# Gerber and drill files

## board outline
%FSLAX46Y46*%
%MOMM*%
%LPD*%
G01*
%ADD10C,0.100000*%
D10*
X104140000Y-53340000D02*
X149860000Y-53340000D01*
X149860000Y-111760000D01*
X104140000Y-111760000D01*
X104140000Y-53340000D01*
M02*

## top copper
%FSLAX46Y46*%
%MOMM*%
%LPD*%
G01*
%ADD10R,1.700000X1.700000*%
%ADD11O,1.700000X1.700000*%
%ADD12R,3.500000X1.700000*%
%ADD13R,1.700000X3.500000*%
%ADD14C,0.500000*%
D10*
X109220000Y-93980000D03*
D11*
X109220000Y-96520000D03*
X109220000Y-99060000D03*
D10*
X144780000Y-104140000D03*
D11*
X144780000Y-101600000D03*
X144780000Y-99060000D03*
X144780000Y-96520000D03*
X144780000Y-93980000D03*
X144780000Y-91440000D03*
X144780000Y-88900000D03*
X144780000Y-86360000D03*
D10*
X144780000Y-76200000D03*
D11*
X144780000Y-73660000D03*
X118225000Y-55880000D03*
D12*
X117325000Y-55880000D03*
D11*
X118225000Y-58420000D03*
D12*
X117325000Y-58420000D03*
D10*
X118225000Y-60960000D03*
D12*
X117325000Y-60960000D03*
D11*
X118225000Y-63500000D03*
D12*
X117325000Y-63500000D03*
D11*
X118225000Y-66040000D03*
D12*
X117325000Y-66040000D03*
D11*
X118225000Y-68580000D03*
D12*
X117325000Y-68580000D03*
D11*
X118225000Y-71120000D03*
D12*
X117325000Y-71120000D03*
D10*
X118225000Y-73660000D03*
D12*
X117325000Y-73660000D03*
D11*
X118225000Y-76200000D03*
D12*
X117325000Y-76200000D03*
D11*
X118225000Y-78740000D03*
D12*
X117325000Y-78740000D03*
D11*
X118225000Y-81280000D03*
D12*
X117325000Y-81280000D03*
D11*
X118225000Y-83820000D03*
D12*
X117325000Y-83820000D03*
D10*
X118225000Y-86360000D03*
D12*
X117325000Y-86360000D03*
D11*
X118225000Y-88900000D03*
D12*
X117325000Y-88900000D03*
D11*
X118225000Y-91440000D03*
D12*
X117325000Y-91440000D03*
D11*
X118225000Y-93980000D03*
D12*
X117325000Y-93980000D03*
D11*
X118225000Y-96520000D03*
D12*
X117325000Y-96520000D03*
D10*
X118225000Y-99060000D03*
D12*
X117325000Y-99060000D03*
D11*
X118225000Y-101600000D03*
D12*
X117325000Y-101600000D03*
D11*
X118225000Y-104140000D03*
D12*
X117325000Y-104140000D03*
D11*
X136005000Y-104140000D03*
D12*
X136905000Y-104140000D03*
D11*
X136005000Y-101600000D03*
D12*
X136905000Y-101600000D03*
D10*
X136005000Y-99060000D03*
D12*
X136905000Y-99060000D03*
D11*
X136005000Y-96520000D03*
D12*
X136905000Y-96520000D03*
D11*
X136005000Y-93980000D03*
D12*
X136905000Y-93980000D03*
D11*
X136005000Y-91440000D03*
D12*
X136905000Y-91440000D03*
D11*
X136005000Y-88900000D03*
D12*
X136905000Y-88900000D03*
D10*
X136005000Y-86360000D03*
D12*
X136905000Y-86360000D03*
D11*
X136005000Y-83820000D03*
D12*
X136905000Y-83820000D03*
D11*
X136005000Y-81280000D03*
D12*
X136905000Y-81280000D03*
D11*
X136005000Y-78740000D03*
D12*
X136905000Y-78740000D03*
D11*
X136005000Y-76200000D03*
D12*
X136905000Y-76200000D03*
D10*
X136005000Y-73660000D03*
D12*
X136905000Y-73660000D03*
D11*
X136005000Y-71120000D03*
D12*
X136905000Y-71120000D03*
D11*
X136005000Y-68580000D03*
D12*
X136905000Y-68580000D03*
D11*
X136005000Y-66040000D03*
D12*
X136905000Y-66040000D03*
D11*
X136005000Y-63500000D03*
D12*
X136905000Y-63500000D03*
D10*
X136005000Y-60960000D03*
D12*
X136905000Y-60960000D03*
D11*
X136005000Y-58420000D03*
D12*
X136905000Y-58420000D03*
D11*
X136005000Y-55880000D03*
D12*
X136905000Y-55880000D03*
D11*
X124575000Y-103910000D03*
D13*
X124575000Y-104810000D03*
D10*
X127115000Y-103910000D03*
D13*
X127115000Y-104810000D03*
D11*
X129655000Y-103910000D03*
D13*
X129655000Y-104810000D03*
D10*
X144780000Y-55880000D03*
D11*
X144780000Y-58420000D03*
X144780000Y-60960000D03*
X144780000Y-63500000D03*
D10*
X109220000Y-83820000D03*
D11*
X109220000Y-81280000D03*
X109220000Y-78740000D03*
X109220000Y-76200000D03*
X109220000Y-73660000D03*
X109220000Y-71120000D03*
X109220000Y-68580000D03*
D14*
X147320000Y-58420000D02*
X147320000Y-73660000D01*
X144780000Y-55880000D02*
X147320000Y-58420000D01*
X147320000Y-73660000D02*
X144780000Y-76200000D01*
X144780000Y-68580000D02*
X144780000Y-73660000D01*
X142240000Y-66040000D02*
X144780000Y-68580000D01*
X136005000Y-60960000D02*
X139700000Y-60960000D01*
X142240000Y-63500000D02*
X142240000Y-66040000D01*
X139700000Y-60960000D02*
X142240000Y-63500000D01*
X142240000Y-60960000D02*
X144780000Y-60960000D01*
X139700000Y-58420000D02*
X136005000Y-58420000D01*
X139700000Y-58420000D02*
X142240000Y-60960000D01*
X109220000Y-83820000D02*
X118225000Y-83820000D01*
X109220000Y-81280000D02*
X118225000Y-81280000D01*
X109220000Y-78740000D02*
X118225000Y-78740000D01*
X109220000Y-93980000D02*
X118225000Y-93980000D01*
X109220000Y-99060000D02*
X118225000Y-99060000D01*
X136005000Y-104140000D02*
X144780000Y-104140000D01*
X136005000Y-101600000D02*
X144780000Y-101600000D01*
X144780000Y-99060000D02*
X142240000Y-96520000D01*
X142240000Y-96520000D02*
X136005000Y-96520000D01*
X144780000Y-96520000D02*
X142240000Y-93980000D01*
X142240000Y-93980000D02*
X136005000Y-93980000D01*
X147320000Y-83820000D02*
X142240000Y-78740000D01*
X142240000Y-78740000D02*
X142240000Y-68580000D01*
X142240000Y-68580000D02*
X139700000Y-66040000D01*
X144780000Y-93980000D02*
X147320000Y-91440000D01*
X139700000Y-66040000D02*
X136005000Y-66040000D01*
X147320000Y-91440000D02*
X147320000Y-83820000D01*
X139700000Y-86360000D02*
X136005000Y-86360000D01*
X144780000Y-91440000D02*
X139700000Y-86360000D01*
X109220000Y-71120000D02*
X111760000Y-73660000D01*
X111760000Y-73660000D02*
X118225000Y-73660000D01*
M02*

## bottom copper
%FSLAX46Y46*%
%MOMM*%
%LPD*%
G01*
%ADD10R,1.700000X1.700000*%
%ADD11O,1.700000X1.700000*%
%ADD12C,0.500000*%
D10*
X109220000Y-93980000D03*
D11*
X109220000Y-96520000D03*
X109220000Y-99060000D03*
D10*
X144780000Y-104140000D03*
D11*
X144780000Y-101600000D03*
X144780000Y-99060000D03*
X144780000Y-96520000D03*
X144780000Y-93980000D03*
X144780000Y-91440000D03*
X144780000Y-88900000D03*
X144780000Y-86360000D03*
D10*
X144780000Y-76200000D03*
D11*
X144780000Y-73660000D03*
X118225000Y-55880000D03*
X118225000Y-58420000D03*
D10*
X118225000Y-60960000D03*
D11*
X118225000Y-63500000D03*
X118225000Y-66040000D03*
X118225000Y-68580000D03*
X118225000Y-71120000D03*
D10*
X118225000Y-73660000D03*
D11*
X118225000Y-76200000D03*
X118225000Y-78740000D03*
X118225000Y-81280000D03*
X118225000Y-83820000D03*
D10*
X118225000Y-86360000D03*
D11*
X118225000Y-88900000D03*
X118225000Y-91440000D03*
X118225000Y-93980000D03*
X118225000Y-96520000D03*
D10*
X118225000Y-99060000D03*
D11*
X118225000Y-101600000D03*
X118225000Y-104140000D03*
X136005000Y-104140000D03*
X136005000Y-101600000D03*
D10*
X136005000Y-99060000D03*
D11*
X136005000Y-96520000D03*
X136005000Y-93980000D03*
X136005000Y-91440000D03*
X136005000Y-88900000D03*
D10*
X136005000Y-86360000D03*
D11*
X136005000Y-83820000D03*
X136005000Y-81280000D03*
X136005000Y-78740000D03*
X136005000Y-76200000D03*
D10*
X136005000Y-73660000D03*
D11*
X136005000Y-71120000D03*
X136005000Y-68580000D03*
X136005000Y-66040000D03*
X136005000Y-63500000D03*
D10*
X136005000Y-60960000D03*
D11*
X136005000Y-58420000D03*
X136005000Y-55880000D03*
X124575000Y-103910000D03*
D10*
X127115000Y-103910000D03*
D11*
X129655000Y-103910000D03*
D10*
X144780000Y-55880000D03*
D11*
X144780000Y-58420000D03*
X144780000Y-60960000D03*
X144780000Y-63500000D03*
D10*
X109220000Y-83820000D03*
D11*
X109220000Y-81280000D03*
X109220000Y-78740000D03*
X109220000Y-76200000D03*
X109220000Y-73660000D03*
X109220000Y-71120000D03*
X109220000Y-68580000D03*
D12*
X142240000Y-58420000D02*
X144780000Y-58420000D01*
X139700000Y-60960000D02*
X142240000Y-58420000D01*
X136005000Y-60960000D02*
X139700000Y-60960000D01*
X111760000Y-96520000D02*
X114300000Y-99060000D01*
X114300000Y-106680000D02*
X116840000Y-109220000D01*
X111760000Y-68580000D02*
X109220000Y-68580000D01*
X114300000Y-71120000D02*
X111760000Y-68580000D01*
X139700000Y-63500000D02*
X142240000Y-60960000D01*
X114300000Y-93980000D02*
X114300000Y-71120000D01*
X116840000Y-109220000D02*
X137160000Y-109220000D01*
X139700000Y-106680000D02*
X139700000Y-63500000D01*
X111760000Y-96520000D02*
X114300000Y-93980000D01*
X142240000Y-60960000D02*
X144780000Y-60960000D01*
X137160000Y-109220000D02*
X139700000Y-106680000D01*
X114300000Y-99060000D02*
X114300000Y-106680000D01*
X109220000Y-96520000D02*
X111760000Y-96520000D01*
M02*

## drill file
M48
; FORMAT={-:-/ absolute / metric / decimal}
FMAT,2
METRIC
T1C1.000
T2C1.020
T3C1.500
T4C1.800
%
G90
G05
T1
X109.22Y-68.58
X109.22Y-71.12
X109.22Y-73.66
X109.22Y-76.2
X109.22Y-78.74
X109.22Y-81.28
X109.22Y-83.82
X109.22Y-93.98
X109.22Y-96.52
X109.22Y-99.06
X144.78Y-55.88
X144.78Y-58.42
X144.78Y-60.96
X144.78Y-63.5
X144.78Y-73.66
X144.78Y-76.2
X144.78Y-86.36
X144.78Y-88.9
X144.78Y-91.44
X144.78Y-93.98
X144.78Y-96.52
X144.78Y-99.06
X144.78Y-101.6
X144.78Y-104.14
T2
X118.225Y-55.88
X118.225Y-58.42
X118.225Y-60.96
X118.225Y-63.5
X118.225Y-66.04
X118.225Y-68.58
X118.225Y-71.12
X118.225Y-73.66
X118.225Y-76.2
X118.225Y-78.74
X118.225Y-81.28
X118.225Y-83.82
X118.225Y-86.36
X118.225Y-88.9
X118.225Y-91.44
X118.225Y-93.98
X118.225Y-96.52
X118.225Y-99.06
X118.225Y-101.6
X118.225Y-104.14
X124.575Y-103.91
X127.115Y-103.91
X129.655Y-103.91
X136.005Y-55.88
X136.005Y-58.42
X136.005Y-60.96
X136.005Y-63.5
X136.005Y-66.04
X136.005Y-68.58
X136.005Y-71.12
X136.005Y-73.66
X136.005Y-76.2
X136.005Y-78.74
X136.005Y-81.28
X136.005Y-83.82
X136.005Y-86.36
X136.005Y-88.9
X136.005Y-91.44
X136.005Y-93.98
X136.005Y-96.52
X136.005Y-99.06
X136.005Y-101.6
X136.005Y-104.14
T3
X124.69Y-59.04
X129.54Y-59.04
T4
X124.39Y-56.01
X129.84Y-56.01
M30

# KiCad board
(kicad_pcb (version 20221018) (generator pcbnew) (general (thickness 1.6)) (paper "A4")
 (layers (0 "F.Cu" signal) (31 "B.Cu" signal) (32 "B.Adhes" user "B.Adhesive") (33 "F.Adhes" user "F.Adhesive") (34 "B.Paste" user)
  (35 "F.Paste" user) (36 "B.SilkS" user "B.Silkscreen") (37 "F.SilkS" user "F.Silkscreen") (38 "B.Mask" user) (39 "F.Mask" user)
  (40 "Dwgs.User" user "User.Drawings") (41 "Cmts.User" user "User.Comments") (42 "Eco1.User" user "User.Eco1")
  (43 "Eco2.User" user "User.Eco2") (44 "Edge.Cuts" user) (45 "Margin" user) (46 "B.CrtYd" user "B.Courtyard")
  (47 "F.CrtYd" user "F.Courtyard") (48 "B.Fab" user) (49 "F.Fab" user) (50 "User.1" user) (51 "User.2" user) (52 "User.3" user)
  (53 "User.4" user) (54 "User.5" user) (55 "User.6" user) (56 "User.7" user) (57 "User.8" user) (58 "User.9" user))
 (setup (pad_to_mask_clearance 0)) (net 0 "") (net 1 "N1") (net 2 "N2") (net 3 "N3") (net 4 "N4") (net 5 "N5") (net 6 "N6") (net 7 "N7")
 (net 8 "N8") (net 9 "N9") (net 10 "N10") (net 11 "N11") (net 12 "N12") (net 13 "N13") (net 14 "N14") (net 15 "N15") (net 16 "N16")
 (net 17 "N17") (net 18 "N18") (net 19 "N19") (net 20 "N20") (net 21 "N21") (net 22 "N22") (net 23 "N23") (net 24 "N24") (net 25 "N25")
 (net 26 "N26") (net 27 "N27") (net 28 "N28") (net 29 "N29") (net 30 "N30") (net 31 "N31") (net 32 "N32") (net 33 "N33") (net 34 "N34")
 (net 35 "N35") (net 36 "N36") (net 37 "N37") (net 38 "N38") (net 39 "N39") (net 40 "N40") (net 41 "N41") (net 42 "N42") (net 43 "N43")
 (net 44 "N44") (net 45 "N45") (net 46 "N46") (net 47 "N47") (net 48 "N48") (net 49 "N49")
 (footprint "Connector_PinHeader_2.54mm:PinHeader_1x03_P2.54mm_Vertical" (layer "F.Cu") (at 109.22 93.98)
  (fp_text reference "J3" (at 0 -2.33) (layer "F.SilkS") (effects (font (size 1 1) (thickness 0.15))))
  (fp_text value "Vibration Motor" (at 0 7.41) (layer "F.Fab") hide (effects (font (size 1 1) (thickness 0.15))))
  (pad "1" thru_hole rect (at 0 0) (size 1.7 1.7) (drill 1) (layers "*.Cu" "*.Mask") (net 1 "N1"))
  (pad "2" thru_hole oval (at 0 2.54) (size 1.7 1.7) (drill 1) (layers "*.Cu" "*.Mask") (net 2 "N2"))
  (pad "3" thru_hole oval (at 0 5.08) (size 1.7 1.7) (drill 1) (layers "*.Cu" "*.Mask") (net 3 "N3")))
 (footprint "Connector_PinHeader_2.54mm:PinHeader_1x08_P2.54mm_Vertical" (layer "F.Cu") (at 144.78 104.14 180)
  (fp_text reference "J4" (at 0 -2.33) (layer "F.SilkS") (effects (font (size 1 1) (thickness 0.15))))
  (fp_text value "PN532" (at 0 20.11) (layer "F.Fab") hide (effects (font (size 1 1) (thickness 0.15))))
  (pad "1" thru_hole rect (at 0 0 180) (size 1.7 1.7) (drill 1) (layers "*.Cu" "*.Mask") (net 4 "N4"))
  (pad "2" thru_hole oval (at 0 2.54 180) (size 1.7 1.7) (drill 1) (layers "*.Cu" "*.Mask") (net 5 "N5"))
  (pad "3" thru_hole oval (at 0 5.08 180) (size 1.7 1.7) (drill 1) (layers "*.Cu" "*.Mask") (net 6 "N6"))
  (pad "4" thru_hole oval (at 0 7.62 180) (size 1.7 1.7) (drill 1) (layers "*.Cu" "*.Mask") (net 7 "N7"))
  (pad "5" thru_hole oval (at 0 10.16 180) (size 1.7 1.7) (drill 1) (layers "*.Cu" "*.Mask") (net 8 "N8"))
  (pad "6" thru_hole oval (at 0 12.7 180) (size 1.7 1.7) (drill 1) (layers "*.Cu" "*.Mask") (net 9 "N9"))
  (pad "7" thru_hole oval (at 0 15.24 180) (size 1.7 1.7) (drill 1) (layers "*.Cu" "*.Mask") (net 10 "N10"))
  (pad "8" thru_hole oval (at 0 17.78 180) (size 1.7 1.7) (drill 1) (layers "*.Cu" "*.Mask") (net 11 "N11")))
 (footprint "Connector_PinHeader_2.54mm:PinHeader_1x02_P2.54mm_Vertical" (layer "F.Cu") (at 144.78 76.2 180)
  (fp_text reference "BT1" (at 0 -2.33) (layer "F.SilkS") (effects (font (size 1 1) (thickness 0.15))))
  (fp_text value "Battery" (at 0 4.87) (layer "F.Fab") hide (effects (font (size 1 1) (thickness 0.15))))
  (pad "1" thru_hole rect (at 0 0 180) (size 1.7 1.7) (drill 1) (layers "*.Cu" "*.Mask") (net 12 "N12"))
  (pad "2" thru_hole oval (at 0 2.54 180) (size 1.7 1.7) (drill 1) (layers "*.Cu" "*.Mask") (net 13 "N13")))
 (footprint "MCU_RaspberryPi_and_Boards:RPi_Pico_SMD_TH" (layer "F.Cu") (at 127.115 80.01)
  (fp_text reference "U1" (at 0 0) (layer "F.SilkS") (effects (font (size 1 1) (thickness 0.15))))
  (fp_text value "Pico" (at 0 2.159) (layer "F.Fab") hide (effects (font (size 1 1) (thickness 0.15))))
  (pad "" np_thru_hole oval (at -2.725 -24) (size 1.8 1.8) (drill 1.8) (layers "*.Cu" "*.Mask"))
  (pad "" np_thru_hole oval (at -2.425 -20.97) (size 1.5 1.5) (drill 1.5) (layers "*.Cu" "*.Mask"))
  (pad "" np_thru_hole oval (at 2.425 -20.97) (size 1.5 1.5) (drill 1.5) (layers "*.Cu" "*.Mask"))
  (pad "" np_thru_hole oval (at 2.725 -24) (size 1.8 1.8) (drill 1.8) (layers "*.Cu" "*.Mask"))
  (pad "1" thru_hole oval (at -8.89 -24.13) (size 1.7 1.7) (drill 1.02) (layers "*.Cu" "*.Mask") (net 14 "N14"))
  (pad "1" smd rect (at -8.89 -24.13) (size 3.5 1.7) (drill (offset -0.9 0)) (layers "F.Cu" "F.Mask") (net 14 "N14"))
  (pad "2" thru_hole oval (at -8.89 -21.59) (size 1.7 1.7) (drill 1.02) (layers "*.Cu" "*.Mask") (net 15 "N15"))
  (pad "2" smd rect (at -8.89 -21.59) (size 3.5 1.7) (drill (offset -0.9 0)) (layers "F.Cu" "F.Mask") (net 15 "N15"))
  (pad "3" thru_hole rect (at -8.89 -19.05) (size 1.7 1.7) (drill 1.02) (layers "*.Cu" "*.Mask") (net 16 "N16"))
  (pad "3" smd rect (at -8.89 -19.05) (size 3.5 1.7) (drill (offset -0.9 0)) (layers "F.Cu" "F.Mask") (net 16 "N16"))
  (pad "4" thru_hole oval (at -8.89 -16.51) (size 1.7 1.7) (drill 1.02) (layers "*.Cu" "*.Mask") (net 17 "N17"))
  (pad "4" smd rect (at -8.89 -16.51) (size 3.5 1.7) (drill (offset -0.9 0)) (layers "F.Cu" "F.Mask") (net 17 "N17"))
  (pad "5" thru_hole oval (at -8.89 -13.97) (size 1.7 1.7) (drill 1.02) (layers "*.Cu" "*.Mask") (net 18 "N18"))
  (pad "5" smd rect (at -8.89 -13.97) (size 3.5 1.7) (drill (offset -0.9 0)) (layers "F.Cu" "F.Mask") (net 18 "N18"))
  (pad "6" thru_hole oval (at -8.89 -11.43) (size 1.7 1.7) (drill 1.02) (layers "*.Cu" "*.Mask") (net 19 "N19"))
  (pad "6" smd rect (at -8.89 -11.43) (size 3.5 1.7) (drill (offset -0.9 0)) (layers "F.Cu" "F.Mask") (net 19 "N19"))
  (pad "7" thru_hole oval (at -8.89 -8.89) (size 1.7 1.7) (drill 1.02) (layers "*.Cu" "*.Mask") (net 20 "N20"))
  (pad "7" smd rect (at -8.89 -8.89) (size 3.5 1.7) (drill (offset -0.9 0)) (layers "F.Cu" "F.Mask") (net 20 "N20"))
  (pad "8" thru_hole rect (at -8.89 -6.35) (size 1.7 1.7) (drill 1.02) (layers "*.Cu" "*.Mask") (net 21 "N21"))
  (pad "8" smd rect (at -8.89 -6.35) (size 3.5 1.7) (drill (offset -0.9 0)) (layers "F.Cu" "F.Mask") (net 21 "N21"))
  (pad "9" thru_hole oval (at -8.89 -3.81) (size 1.7 1.7) (drill 1.02) (layers "*.Cu" "*.Mask") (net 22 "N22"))
  (pad "9" smd rect (at -8.89 -3.81) (size 3.5 1.7) (drill (offset -0.9 0)) (layers "F.Cu" "F.Mask") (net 22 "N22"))
  (pad "10" thru_hole oval (at -8.89 -1.27) (size 1.7 1.7) (drill 1.02) (layers "*.Cu" "*.Mask") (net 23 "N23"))
  (pad "10" smd rect (at -8.89 -1.27) (size 3.5 1.7) (drill (offset -0.9 0)) (layers "F.Cu" "F.Mask") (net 23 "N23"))
  (pad "11" thru_hole oval (at -8.89 1.27) (size 1.7 1.7) (drill 1.02) (layers "*.Cu" "*.Mask") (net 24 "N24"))
  (pad "11" smd rect (at -8.89 1.27) (size 3.5 1.7) (drill (offset -0.9 0)) (layers "F.Cu" "F.Mask") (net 24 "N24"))
  (pad "12" thru_hole oval (at -8.89 3.81) (size 1.7 1.7) (drill 1.02) (layers "*.Cu" "*.Mask") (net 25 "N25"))
  (pad "12" smd rect (at -8.89 3.81) (size 3.5 1.7) (drill (offset -0.9 0)) (layers "F.Cu" "F.Mask") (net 25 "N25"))
  (pad "13" thru_hole rect (at -8.89 6.35) (size 1.7 1.7) (drill 1.02) (layers "*.Cu" "*.Mask") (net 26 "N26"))
  (pad "13" smd rect (at -8.89 6.35) (size 3.5 1.7) (drill (offset -0.9 0)) (layers "F.Cu" "F.Mask") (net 26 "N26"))
  (pad "14" thru_hole oval (at -8.89 8.89) (size 1.7 1.7) (drill 1.02) (layers "*.Cu" "*.Mask") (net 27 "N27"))
  (pad "14" smd rect (at -8.89 8.89) (size 3.5 1.7) (drill (offset -0.9 0)) (layers "F.Cu" "F.Mask") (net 27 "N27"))
  (pad "15" thru_hole oval (at -8.89 11.43) (size 1.7 1.7) (drill 1.02) (layers "*.Cu" "*.Mask") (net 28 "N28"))
  (pad "15" smd rect (at -8.89 11.43) (size 3.5 1.7) (drill (offset -0.9 0)) (layers "F.Cu" "F.Mask") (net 28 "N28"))
  (pad "16" thru_hole oval (at -8.89 13.97) (size 1.7 1.7) (drill 1.02) (layers "*.Cu" "*.Mask") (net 1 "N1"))
  (pad "16" smd rect (at -8.89 13.97) (size 3.5 1.7) (drill (offset -0.9 0)) (layers "F.Cu" "F.Mask") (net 1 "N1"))
  (pad "17" thru_hole oval (at -8.89 16.51) (size 1.7 1.7) (drill 1.02) (layers "*.Cu" "*.Mask") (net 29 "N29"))
  (pad "17" smd rect (at -8.89 16.51) (size 3.5 1.7) (drill (offset -0.9 0)) (layers "F.Cu" "F.Mask") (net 29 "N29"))
  (pad "18" thru_hole rect (at -8.89 19.05) (size 1.7 1.7) (drill 1.02) (layers "*.Cu" "*.Mask") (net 3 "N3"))
  (pad "18" smd rect (at -8.89 19.05) (size 3.5 1.7) (drill (offset -0.9 0)) (layers "F.Cu" "F.Mask") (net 3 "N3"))
  (pad "19" thru_hole oval (at -8.89 21.59) (size 1.7 1.7) (drill 1.02) (layers "*.Cu" "*.Mask") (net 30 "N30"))
  (pad "19" smd rect (at -8.89 21.59) (size 3.5 1.7) (drill (offset -0.9 0)) (layers "F.Cu" "F.Mask") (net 30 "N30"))
  (pad "20" thru_hole oval (at -8.89 24.13) (size 1.7 1.7) (drill 1.02) (layers "*.Cu" "*.Mask") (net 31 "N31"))
  (pad "20" smd rect (at -8.89 24.13) (size 3.5 1.7) (drill (offset -0.9 0)) (layers "F.Cu" "F.Mask") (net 31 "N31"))
  (pad "21" thru_hole oval (at 8.89 24.13) (size 1.7 1.7) (drill 1.02) (layers "*.Cu" "*.Mask") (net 4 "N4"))
  (pad "21" smd rect (at 8.89 24.13) (size 3.5 1.7) (drill (offset 0.9 0)) (layers "F.Cu" "F.Mask") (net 4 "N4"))
  (pad "22" thru_hole oval (at 8.89 21.59) (size 1.7 1.7) (drill 1.02) (layers "*.Cu" "*.Mask") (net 5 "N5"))
  (pad "22" smd rect (at 8.89 21.59) (size 3.5 1.7) (drill (offset 0.9 0)) (layers "F.Cu" "F.Mask") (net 5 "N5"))
  (pad "23" thru_hole rect (at 8.89 19.05) (size 1.7 1.7) (drill 1.02) (layers "*.Cu" "*.Mask") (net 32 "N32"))
  (pad "23" smd rect (at 8.89 19.05) (size 3.5 1.7) (drill (offset 0.9 0)) (layers "F.Cu" "F.Mask") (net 32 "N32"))
  (pad "24" thru_hole oval (at 8.89 16.51) (size 1.7 1.7) (drill 1.02) (layers "*.Cu" "*.Mask") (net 6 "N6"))
  (pad "24" smd rect (at 8.89 16.51) (size 3.5 1.7) (drill (offset 0.9 0)) (layers "F.Cu" "F.Mask") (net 6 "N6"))
  (pad "25" thru_hole oval (at 8.89 13.97) (size 1.7 1.7) (drill 1.02) (layers "*.Cu" "*.Mask") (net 7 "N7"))
  (pad "25" smd rect (at 8.89 13.97) (size 3.5 1.7) (drill (offset 0.9 0)) (layers "F.Cu" "F.Mask") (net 7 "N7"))
  (pad "26" thru_hole oval (at 8.89 11.43) (size 1.7 1.7) (drill 1.02) (layers "*.Cu" "*.Mask") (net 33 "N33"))
  (pad "26" smd rect (at 8.89 11.43) (size 3.5 1.7) (drill (offset 0.9 0)) (layers "F.Cu" "F.Mask") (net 33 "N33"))
  (pad "27" thru_hole oval (at 8.89 8.89) (size 1.7 1.7) (drill 1.02) (layers "*.Cu" "*.Mask") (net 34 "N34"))
  (pad "27" smd rect (at 8.89 8.89) (size 3.5 1.7) (drill (offset 0.9 0)) (layers "F.Cu" "F.Mask") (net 34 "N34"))
  (pad "28" thru_hole rect (at 8.89 6.35) (size 1.7 1.7) (drill 1.02) (layers "*.Cu" "*.Mask") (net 9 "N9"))
  (pad "28" smd rect (at 8.89 6.35) (size 3.5 1.7) (drill (offset 0.9 0)) (layers "F.Cu" "F.Mask") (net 9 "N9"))
  (pad "29" thru_hole oval (at 8.89 3.81) (size 1.7 1.7) (drill 1.02) (layers "*.Cu" "*.Mask") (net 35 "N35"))
  (pad "29" smd rect (at 8.89 3.81) (size 3.5 1.7) (drill (offset 0.9 0)) (layers "F.Cu" "F.Mask") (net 35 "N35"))
  (pad "30" thru_hole oval (at 8.89 1.27) (size 1.7 1.7) (drill 1.02) (layers "*.Cu" "*.Mask") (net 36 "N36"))
  (pad "30" smd rect (at 8.89 1.27) (size 3.5 1.7) (drill (offset 0.9 0)) (layers "F.Cu" "F.Mask") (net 36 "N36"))
  (pad "31" thru_hole oval (at 8.89 -1.27) (size 1.7 1.7) (drill 1.02) (layers "*.Cu" "*.Mask") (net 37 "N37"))
  (pad "31" smd rect (at 8.89 -1.27) (size 3.5 1.7) (drill (offset 0.9 0)) (layers "F.Cu" "F.Mask") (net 37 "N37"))
  (pad "32" thru_hole oval (at 8.89 -3.81) (size 1.7 1.7) (drill 1.02) (layers "*.Cu" "*.Mask") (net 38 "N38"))
  (pad "32" smd rect (at 8.89 -3.81) (size 3.5 1.7) (drill (offset 0.9 0)) (layers "F.Cu" "F.Mask") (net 38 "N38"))
  (pad "33" thru_hole rect (at 8.89 -6.35) (size 1.7 1.7) (drill 1.02) (layers "*.Cu" "*.Mask") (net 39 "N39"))
  (pad "33" smd rect (at 8.89 -6.35) (size 3.5 1.7) (drill (offset 0.9 0)) (layers "F.Cu" "F.Mask") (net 39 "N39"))
  (pad "34" thru_hole oval (at 8.89 -8.89) (size 1.7 1.7) (drill 1.02) (layers "*.Cu" "*.Mask") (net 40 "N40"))
  (pad "34" smd rect (at 8.89 -8.89) (size 3.5 1.7) (drill (offset 0.9 0)) (layers "F.Cu" "F.Mask") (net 40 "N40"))
  (pad "35" thru_hole oval (at 8.89 -11.43) (size 1.7 1.7) (drill 1.02) (layers "*.Cu" "*.Mask") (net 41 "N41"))
  (pad "35" smd rect (at 8.89 -11.43) (size 3.5 1.7) (drill (offset 0.9 0)) (layers "F.Cu" "F.Mask") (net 41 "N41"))
  (pad "36" thru_hole oval (at 8.89 -13.97) (size 1.7 1.7) (drill 1.02) (layers "*.Cu" "*.Mask") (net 8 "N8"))
  (pad "36" smd rect (at 8.89 -13.97) (size 3.5 1.7) (drill (offset 0.9 0)) (layers "F.Cu" "F.Mask") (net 8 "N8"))
  (pad "37" thru_hole oval (at 8.89 -16.51) (size 1.7 1.7) (drill 1.02) (layers "*.Cu" "*.Mask") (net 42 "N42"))
  (pad "37" smd rect (at 8.89 -16.51) (size 3.5 1.7) (drill (offset 0.9 0)) (layers "F.Cu" "F.Mask") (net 42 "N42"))
  (pad "38" thru_hole rect (at 8.89 -19.05) (size 1.7 1.7) (drill 1.02) (layers "*.Cu" "*.Mask") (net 13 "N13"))
  (pad "38" smd rect (at 8.89 -19.05) (size 3.5 1.7) (drill (offset 0.9 0)) (layers "F.Cu" "F.Mask") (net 13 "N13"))
  (pad "39" thru_hole oval (at 8.89 -21.59) (size 1.7 1.7) (drill 1.02) (layers "*.Cu" "*.Mask") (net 2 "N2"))
  (pad "39" smd rect (at 8.89 -21.59) (size 3.5 1.7) (drill (offset 0.9 0)) (layers "F.Cu" "F.Mask") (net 2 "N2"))
  (pad "40" thru_hole oval (at 8.89 -24.13) (size 1.7 1.7) (drill 1.02) (layers "*.Cu" "*.Mask") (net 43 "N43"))
  (pad "40" smd rect (at 8.89 -24.13) (size 3.5 1.7) (drill (offset 0.9 0)) (layers "F.Cu" "F.Mask") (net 43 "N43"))
  (pad "41" thru_hole oval (at -2.54 23.9) (size 1.7 1.7) (drill 1.02) (layers "*.Cu" "*.Mask") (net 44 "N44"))
  (pad "41" smd rect (at -2.54 23.9 90) (size 3.5 1.7) (drill (offset -0.9 0)) (layers "F.Cu" "F.Mask") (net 44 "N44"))
  (pad "42" thru_hole rect (at 0 23.9) (size 1.7 1.7) (drill 1.02) (layers "*.Cu" "*.Mask") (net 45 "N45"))
  (pad "42" smd rect (at 0 23.9 90) (size 3.5 1.7) (drill (offset -0.9 0)) (layers "F.Cu" "F.Mask") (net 45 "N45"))
  (pad "43" thru_hole oval (at 2.54 23.9) (size 1.7 1.7) (drill 1.02) (layers "*.Cu" "*.Mask") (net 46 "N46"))
  (pad "43" smd rect (at 2.54 23.9 90) (size 3.5 1.7) (drill (offset -0.9 0)) (layers "F.Cu" "F.Mask") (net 46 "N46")))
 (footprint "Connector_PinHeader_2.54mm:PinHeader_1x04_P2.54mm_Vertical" (layer "F.Cu") (at 144.78 55.88)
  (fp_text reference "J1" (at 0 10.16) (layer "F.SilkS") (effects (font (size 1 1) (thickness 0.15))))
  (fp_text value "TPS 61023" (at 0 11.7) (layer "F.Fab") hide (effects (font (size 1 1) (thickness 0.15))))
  (pad "1" thru_hole rect (at 0 0) (size 1.7 1.7) (drill 1) (layers "*.Cu" "*.Mask") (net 12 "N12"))
  (pad "2" thru_hole oval (at 0 2.54) (size 1.7 1.7) (drill 1) (layers "*.Cu" "*.Mask") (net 13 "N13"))
  (pad "3" thru_hole oval (at 0 5.08) (size 1.7 1.7) (drill 1) (layers "*.Cu" "*.Mask") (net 2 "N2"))
  (pad "4" thru_hole oval (at 0 7.62) (size 1.7 1.7) (drill 1) (layers "*.Cu" "*.Mask") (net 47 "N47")))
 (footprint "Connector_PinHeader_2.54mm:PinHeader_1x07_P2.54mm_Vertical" (layer "F.Cu") (at 109.22 83.82 180)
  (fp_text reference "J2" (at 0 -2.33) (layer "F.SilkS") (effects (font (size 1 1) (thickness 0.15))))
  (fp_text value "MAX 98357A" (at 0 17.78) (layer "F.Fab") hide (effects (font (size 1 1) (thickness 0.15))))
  (pad "1" thru_hole rect (at 0 0 180) (size 1.7 1.7) (drill 1) (layers "*.Cu" "*.Mask") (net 25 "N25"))
  (pad "2" thru_hole oval (at 0 2.54 180) (size 1.7 1.7) (drill 1) (layers "*.Cu" "*.Mask") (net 24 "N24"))
  (pad "3" thru_hole oval (at 0 5.08 180) (size 1.7 1.7) (drill 1) (layers "*.Cu" "*.Mask") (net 23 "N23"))
  (pad "4" thru_hole oval (at 0 7.62 180) (size 1.7 1.7) (drill 1) (layers "*.Cu" "*.Mask") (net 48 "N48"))
  (pad "5" thru_hole oval (at 0 10.16 180) (size 1.7 1.7) (drill 1) (layers "*.Cu" "*.Mask") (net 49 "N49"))
  (pad "6" thru_hole oval (at 0 12.7 180) (size 1.7 1.7) (drill 1) (layers "*.Cu" "*.Mask") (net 21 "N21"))
  (pad "7" thru_hole oval (at 0 15.24 180) (size 1.7 1.7) (drill 1) (layers "*.Cu" "*.Mask") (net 2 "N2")))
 (gr_rect (start 104.14 53.34) (end 149.86 111.76) (stroke (width 0.1) (type default)) (fill none) (layer "Edge.Cuts"))
 (segment (start 147.32 58.42) (end 147.32 73.66) (width 0.5) (layer "F.Cu") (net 12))
 (segment (start 144.78 55.88) (end 147.32 58.42) (width 0.5) (layer "F.Cu") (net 12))
 (segment (start 147.32 73.66) (end 144.78 76.2) (width 0.5) (layer "F.Cu") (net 12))
 (segment (start 144.78 68.58) (end 144.78 73.66) (width 0.5) (layer "F.Cu") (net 13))
 (segment (start 142.24 66.04) (end 144.78 68.58) (width 0.5) (layer "F.Cu") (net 13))
 (segment (start 136.005 60.96) (end 139.7 60.96) (width 0.5) (layer "F.Cu") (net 13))
 (segment (start 142.24 63.5) (end 142.24 66.04) (width 0.5) (layer "F.Cu") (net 13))
 (segment (start 139.7 60.96) (end 142.24 63.5) (width 0.5) (layer "F.Cu") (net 13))
 (segment (start 142.24 58.42) (end 144.78 58.42) (width 0.5) (layer "B.Cu") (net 13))
 (segment (start 139.7 60.96) (end 142.24 58.42) (width 0.5) (layer "B.Cu") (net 13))
 (segment (start 136.005 60.96) (end 139.7 60.96) (width 0.5) (layer "B.Cu") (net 13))
 (segment (start 142.24 60.96) (end 144.78 60.96) (width 0.5) (layer "F.Cu") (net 2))
 (segment (start 139.7 58.42) (end 136.005 58.42) (width 0.5) (layer "F.Cu") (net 2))
 (segment (start 139.7 58.42) (end 142.24 60.96) (width 0.5) (layer "F.Cu") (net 2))
 (segment (start 111.76 96.52) (end 114.3 99.06) (width 0.5) (layer "B.Cu") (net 2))
 (segment (start 114.3 106.68) (end 116.84 109.22) (width 0.5) (layer "B.Cu") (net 2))
 (segment (start 111.76 68.58) (end 109.22 68.58) (width 0.5) (layer "B.Cu") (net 2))
 (segment (start 114.3 71.12) (end 111.76 68.58) (width 0.5) (layer "B.Cu") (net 2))
 (segment (start 139.7 63.5) (end 142.24 60.96) (width 0.5) (layer "B.Cu") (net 2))
 (segment (start 114.3 93.98) (end 114.3 71.12) (width 0.5) (layer "B.Cu") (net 2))
 (segment (start 116.84 109.22) (end 137.16 109.22) (width 0.5) (layer "B.Cu") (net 2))
 (segment (start 139.7 106.68) (end 139.7 63.5) (width 0.5) (layer "B.Cu") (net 2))
 (segment (start 111.76 96.52) (end 114.3 93.98) (width 0.5) (layer "B.Cu") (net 2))
 (segment (start 142.24 60.96) (end 144.78 60.96) (width 0.5) (layer "B.Cu") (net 2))
 (segment (start 137.16 109.22) (end 139.7 106.68) (width 0.5) (layer "B.Cu") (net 2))
 (segment (start 114.3 99.06) (end 114.3 106.68) (width 0.5) (layer "B.Cu") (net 2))
 (segment (start 109.22 96.52) (end 111.76 96.52) (width 0.5) (layer "B.Cu") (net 2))
 (segment (start 109.22 83.82) (end 118.225 83.82) (width 0.5) (layer "F.Cu") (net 25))
 (segment (start 109.22 81.28) (end 118.225 81.28) (width 0.5) (layer "F.Cu") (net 24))
 (segment (start 109.22 78.74) (end 118.225 78.74) (width 0.5) (layer "F.Cu") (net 23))
 (segment (start 109.22 93.98) (end 118.225 93.98) (width 0.5) (layer "F.Cu") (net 1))
 (segment (start 109.22 99.06) (end 118.225 99.06) (width 0.5) (layer "F.Cu") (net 3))
 (segment (start 136.005 104.14) (end 144.78 104.14) (width 0.5) (layer "F.Cu") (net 4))
 (segment (start 136.005 101.6) (end 144.78 101.6) (width 0.5) (layer "F.Cu") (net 5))
 (segment (start 144.78 99.06) (end 142.24 96.52) (width 0.5) (layer "F.Cu") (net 6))
 (segment (start 142.24 96.52) (end 136.005 96.52) (width 0.5) (layer "F.Cu") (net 6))
 (segment (start 144.78 96.52) (end 142.24 93.98) (width 0.5) (layer "F.Cu") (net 7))
 (segment (start 142.24 93.98) (end 136.005 93.98) (width 0.5) (layer "F.Cu") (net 7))
 (segment (start 147.32 83.82) (end 142.24 78.74) (width 0.5) (layer "F.Cu") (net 8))
 (segment (start 142.24 78.74) (end 142.24 68.58) (width 0.5) (layer "F.Cu") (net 8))
 (segment (start 142.24 68.58) (end 139.7 66.04) (width 0.5) (layer "F.Cu") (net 8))
 (segment (start 144.78 93.98) (end 147.32 91.44) (width 0.5) (layer "F.Cu") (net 8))
 (segment (start 139.7 66.04) (end 136.005 66.04) (width 0.5) (layer "F.Cu") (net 8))
 (segment (start 147.32 91.44) (end 147.32 83.82) (width 0.5) (layer "F.Cu") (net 8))
 (segment (start 139.7 86.36) (end 136.005 86.36) (width 0.5) (layer "F.Cu") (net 9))
 (segment (start 144.78 91.44) (end 139.7 86.36) (width 0.5) (layer "F.Cu") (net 9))
 (segment (start 109.22 71.12) (end 111.76 73.66) (width 0.5) (layer "F.Cu") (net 21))
 (segment (start 111.76 73.66) (end 118.225 73.66) (width 0.5) (layer "F.Cu") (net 21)))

